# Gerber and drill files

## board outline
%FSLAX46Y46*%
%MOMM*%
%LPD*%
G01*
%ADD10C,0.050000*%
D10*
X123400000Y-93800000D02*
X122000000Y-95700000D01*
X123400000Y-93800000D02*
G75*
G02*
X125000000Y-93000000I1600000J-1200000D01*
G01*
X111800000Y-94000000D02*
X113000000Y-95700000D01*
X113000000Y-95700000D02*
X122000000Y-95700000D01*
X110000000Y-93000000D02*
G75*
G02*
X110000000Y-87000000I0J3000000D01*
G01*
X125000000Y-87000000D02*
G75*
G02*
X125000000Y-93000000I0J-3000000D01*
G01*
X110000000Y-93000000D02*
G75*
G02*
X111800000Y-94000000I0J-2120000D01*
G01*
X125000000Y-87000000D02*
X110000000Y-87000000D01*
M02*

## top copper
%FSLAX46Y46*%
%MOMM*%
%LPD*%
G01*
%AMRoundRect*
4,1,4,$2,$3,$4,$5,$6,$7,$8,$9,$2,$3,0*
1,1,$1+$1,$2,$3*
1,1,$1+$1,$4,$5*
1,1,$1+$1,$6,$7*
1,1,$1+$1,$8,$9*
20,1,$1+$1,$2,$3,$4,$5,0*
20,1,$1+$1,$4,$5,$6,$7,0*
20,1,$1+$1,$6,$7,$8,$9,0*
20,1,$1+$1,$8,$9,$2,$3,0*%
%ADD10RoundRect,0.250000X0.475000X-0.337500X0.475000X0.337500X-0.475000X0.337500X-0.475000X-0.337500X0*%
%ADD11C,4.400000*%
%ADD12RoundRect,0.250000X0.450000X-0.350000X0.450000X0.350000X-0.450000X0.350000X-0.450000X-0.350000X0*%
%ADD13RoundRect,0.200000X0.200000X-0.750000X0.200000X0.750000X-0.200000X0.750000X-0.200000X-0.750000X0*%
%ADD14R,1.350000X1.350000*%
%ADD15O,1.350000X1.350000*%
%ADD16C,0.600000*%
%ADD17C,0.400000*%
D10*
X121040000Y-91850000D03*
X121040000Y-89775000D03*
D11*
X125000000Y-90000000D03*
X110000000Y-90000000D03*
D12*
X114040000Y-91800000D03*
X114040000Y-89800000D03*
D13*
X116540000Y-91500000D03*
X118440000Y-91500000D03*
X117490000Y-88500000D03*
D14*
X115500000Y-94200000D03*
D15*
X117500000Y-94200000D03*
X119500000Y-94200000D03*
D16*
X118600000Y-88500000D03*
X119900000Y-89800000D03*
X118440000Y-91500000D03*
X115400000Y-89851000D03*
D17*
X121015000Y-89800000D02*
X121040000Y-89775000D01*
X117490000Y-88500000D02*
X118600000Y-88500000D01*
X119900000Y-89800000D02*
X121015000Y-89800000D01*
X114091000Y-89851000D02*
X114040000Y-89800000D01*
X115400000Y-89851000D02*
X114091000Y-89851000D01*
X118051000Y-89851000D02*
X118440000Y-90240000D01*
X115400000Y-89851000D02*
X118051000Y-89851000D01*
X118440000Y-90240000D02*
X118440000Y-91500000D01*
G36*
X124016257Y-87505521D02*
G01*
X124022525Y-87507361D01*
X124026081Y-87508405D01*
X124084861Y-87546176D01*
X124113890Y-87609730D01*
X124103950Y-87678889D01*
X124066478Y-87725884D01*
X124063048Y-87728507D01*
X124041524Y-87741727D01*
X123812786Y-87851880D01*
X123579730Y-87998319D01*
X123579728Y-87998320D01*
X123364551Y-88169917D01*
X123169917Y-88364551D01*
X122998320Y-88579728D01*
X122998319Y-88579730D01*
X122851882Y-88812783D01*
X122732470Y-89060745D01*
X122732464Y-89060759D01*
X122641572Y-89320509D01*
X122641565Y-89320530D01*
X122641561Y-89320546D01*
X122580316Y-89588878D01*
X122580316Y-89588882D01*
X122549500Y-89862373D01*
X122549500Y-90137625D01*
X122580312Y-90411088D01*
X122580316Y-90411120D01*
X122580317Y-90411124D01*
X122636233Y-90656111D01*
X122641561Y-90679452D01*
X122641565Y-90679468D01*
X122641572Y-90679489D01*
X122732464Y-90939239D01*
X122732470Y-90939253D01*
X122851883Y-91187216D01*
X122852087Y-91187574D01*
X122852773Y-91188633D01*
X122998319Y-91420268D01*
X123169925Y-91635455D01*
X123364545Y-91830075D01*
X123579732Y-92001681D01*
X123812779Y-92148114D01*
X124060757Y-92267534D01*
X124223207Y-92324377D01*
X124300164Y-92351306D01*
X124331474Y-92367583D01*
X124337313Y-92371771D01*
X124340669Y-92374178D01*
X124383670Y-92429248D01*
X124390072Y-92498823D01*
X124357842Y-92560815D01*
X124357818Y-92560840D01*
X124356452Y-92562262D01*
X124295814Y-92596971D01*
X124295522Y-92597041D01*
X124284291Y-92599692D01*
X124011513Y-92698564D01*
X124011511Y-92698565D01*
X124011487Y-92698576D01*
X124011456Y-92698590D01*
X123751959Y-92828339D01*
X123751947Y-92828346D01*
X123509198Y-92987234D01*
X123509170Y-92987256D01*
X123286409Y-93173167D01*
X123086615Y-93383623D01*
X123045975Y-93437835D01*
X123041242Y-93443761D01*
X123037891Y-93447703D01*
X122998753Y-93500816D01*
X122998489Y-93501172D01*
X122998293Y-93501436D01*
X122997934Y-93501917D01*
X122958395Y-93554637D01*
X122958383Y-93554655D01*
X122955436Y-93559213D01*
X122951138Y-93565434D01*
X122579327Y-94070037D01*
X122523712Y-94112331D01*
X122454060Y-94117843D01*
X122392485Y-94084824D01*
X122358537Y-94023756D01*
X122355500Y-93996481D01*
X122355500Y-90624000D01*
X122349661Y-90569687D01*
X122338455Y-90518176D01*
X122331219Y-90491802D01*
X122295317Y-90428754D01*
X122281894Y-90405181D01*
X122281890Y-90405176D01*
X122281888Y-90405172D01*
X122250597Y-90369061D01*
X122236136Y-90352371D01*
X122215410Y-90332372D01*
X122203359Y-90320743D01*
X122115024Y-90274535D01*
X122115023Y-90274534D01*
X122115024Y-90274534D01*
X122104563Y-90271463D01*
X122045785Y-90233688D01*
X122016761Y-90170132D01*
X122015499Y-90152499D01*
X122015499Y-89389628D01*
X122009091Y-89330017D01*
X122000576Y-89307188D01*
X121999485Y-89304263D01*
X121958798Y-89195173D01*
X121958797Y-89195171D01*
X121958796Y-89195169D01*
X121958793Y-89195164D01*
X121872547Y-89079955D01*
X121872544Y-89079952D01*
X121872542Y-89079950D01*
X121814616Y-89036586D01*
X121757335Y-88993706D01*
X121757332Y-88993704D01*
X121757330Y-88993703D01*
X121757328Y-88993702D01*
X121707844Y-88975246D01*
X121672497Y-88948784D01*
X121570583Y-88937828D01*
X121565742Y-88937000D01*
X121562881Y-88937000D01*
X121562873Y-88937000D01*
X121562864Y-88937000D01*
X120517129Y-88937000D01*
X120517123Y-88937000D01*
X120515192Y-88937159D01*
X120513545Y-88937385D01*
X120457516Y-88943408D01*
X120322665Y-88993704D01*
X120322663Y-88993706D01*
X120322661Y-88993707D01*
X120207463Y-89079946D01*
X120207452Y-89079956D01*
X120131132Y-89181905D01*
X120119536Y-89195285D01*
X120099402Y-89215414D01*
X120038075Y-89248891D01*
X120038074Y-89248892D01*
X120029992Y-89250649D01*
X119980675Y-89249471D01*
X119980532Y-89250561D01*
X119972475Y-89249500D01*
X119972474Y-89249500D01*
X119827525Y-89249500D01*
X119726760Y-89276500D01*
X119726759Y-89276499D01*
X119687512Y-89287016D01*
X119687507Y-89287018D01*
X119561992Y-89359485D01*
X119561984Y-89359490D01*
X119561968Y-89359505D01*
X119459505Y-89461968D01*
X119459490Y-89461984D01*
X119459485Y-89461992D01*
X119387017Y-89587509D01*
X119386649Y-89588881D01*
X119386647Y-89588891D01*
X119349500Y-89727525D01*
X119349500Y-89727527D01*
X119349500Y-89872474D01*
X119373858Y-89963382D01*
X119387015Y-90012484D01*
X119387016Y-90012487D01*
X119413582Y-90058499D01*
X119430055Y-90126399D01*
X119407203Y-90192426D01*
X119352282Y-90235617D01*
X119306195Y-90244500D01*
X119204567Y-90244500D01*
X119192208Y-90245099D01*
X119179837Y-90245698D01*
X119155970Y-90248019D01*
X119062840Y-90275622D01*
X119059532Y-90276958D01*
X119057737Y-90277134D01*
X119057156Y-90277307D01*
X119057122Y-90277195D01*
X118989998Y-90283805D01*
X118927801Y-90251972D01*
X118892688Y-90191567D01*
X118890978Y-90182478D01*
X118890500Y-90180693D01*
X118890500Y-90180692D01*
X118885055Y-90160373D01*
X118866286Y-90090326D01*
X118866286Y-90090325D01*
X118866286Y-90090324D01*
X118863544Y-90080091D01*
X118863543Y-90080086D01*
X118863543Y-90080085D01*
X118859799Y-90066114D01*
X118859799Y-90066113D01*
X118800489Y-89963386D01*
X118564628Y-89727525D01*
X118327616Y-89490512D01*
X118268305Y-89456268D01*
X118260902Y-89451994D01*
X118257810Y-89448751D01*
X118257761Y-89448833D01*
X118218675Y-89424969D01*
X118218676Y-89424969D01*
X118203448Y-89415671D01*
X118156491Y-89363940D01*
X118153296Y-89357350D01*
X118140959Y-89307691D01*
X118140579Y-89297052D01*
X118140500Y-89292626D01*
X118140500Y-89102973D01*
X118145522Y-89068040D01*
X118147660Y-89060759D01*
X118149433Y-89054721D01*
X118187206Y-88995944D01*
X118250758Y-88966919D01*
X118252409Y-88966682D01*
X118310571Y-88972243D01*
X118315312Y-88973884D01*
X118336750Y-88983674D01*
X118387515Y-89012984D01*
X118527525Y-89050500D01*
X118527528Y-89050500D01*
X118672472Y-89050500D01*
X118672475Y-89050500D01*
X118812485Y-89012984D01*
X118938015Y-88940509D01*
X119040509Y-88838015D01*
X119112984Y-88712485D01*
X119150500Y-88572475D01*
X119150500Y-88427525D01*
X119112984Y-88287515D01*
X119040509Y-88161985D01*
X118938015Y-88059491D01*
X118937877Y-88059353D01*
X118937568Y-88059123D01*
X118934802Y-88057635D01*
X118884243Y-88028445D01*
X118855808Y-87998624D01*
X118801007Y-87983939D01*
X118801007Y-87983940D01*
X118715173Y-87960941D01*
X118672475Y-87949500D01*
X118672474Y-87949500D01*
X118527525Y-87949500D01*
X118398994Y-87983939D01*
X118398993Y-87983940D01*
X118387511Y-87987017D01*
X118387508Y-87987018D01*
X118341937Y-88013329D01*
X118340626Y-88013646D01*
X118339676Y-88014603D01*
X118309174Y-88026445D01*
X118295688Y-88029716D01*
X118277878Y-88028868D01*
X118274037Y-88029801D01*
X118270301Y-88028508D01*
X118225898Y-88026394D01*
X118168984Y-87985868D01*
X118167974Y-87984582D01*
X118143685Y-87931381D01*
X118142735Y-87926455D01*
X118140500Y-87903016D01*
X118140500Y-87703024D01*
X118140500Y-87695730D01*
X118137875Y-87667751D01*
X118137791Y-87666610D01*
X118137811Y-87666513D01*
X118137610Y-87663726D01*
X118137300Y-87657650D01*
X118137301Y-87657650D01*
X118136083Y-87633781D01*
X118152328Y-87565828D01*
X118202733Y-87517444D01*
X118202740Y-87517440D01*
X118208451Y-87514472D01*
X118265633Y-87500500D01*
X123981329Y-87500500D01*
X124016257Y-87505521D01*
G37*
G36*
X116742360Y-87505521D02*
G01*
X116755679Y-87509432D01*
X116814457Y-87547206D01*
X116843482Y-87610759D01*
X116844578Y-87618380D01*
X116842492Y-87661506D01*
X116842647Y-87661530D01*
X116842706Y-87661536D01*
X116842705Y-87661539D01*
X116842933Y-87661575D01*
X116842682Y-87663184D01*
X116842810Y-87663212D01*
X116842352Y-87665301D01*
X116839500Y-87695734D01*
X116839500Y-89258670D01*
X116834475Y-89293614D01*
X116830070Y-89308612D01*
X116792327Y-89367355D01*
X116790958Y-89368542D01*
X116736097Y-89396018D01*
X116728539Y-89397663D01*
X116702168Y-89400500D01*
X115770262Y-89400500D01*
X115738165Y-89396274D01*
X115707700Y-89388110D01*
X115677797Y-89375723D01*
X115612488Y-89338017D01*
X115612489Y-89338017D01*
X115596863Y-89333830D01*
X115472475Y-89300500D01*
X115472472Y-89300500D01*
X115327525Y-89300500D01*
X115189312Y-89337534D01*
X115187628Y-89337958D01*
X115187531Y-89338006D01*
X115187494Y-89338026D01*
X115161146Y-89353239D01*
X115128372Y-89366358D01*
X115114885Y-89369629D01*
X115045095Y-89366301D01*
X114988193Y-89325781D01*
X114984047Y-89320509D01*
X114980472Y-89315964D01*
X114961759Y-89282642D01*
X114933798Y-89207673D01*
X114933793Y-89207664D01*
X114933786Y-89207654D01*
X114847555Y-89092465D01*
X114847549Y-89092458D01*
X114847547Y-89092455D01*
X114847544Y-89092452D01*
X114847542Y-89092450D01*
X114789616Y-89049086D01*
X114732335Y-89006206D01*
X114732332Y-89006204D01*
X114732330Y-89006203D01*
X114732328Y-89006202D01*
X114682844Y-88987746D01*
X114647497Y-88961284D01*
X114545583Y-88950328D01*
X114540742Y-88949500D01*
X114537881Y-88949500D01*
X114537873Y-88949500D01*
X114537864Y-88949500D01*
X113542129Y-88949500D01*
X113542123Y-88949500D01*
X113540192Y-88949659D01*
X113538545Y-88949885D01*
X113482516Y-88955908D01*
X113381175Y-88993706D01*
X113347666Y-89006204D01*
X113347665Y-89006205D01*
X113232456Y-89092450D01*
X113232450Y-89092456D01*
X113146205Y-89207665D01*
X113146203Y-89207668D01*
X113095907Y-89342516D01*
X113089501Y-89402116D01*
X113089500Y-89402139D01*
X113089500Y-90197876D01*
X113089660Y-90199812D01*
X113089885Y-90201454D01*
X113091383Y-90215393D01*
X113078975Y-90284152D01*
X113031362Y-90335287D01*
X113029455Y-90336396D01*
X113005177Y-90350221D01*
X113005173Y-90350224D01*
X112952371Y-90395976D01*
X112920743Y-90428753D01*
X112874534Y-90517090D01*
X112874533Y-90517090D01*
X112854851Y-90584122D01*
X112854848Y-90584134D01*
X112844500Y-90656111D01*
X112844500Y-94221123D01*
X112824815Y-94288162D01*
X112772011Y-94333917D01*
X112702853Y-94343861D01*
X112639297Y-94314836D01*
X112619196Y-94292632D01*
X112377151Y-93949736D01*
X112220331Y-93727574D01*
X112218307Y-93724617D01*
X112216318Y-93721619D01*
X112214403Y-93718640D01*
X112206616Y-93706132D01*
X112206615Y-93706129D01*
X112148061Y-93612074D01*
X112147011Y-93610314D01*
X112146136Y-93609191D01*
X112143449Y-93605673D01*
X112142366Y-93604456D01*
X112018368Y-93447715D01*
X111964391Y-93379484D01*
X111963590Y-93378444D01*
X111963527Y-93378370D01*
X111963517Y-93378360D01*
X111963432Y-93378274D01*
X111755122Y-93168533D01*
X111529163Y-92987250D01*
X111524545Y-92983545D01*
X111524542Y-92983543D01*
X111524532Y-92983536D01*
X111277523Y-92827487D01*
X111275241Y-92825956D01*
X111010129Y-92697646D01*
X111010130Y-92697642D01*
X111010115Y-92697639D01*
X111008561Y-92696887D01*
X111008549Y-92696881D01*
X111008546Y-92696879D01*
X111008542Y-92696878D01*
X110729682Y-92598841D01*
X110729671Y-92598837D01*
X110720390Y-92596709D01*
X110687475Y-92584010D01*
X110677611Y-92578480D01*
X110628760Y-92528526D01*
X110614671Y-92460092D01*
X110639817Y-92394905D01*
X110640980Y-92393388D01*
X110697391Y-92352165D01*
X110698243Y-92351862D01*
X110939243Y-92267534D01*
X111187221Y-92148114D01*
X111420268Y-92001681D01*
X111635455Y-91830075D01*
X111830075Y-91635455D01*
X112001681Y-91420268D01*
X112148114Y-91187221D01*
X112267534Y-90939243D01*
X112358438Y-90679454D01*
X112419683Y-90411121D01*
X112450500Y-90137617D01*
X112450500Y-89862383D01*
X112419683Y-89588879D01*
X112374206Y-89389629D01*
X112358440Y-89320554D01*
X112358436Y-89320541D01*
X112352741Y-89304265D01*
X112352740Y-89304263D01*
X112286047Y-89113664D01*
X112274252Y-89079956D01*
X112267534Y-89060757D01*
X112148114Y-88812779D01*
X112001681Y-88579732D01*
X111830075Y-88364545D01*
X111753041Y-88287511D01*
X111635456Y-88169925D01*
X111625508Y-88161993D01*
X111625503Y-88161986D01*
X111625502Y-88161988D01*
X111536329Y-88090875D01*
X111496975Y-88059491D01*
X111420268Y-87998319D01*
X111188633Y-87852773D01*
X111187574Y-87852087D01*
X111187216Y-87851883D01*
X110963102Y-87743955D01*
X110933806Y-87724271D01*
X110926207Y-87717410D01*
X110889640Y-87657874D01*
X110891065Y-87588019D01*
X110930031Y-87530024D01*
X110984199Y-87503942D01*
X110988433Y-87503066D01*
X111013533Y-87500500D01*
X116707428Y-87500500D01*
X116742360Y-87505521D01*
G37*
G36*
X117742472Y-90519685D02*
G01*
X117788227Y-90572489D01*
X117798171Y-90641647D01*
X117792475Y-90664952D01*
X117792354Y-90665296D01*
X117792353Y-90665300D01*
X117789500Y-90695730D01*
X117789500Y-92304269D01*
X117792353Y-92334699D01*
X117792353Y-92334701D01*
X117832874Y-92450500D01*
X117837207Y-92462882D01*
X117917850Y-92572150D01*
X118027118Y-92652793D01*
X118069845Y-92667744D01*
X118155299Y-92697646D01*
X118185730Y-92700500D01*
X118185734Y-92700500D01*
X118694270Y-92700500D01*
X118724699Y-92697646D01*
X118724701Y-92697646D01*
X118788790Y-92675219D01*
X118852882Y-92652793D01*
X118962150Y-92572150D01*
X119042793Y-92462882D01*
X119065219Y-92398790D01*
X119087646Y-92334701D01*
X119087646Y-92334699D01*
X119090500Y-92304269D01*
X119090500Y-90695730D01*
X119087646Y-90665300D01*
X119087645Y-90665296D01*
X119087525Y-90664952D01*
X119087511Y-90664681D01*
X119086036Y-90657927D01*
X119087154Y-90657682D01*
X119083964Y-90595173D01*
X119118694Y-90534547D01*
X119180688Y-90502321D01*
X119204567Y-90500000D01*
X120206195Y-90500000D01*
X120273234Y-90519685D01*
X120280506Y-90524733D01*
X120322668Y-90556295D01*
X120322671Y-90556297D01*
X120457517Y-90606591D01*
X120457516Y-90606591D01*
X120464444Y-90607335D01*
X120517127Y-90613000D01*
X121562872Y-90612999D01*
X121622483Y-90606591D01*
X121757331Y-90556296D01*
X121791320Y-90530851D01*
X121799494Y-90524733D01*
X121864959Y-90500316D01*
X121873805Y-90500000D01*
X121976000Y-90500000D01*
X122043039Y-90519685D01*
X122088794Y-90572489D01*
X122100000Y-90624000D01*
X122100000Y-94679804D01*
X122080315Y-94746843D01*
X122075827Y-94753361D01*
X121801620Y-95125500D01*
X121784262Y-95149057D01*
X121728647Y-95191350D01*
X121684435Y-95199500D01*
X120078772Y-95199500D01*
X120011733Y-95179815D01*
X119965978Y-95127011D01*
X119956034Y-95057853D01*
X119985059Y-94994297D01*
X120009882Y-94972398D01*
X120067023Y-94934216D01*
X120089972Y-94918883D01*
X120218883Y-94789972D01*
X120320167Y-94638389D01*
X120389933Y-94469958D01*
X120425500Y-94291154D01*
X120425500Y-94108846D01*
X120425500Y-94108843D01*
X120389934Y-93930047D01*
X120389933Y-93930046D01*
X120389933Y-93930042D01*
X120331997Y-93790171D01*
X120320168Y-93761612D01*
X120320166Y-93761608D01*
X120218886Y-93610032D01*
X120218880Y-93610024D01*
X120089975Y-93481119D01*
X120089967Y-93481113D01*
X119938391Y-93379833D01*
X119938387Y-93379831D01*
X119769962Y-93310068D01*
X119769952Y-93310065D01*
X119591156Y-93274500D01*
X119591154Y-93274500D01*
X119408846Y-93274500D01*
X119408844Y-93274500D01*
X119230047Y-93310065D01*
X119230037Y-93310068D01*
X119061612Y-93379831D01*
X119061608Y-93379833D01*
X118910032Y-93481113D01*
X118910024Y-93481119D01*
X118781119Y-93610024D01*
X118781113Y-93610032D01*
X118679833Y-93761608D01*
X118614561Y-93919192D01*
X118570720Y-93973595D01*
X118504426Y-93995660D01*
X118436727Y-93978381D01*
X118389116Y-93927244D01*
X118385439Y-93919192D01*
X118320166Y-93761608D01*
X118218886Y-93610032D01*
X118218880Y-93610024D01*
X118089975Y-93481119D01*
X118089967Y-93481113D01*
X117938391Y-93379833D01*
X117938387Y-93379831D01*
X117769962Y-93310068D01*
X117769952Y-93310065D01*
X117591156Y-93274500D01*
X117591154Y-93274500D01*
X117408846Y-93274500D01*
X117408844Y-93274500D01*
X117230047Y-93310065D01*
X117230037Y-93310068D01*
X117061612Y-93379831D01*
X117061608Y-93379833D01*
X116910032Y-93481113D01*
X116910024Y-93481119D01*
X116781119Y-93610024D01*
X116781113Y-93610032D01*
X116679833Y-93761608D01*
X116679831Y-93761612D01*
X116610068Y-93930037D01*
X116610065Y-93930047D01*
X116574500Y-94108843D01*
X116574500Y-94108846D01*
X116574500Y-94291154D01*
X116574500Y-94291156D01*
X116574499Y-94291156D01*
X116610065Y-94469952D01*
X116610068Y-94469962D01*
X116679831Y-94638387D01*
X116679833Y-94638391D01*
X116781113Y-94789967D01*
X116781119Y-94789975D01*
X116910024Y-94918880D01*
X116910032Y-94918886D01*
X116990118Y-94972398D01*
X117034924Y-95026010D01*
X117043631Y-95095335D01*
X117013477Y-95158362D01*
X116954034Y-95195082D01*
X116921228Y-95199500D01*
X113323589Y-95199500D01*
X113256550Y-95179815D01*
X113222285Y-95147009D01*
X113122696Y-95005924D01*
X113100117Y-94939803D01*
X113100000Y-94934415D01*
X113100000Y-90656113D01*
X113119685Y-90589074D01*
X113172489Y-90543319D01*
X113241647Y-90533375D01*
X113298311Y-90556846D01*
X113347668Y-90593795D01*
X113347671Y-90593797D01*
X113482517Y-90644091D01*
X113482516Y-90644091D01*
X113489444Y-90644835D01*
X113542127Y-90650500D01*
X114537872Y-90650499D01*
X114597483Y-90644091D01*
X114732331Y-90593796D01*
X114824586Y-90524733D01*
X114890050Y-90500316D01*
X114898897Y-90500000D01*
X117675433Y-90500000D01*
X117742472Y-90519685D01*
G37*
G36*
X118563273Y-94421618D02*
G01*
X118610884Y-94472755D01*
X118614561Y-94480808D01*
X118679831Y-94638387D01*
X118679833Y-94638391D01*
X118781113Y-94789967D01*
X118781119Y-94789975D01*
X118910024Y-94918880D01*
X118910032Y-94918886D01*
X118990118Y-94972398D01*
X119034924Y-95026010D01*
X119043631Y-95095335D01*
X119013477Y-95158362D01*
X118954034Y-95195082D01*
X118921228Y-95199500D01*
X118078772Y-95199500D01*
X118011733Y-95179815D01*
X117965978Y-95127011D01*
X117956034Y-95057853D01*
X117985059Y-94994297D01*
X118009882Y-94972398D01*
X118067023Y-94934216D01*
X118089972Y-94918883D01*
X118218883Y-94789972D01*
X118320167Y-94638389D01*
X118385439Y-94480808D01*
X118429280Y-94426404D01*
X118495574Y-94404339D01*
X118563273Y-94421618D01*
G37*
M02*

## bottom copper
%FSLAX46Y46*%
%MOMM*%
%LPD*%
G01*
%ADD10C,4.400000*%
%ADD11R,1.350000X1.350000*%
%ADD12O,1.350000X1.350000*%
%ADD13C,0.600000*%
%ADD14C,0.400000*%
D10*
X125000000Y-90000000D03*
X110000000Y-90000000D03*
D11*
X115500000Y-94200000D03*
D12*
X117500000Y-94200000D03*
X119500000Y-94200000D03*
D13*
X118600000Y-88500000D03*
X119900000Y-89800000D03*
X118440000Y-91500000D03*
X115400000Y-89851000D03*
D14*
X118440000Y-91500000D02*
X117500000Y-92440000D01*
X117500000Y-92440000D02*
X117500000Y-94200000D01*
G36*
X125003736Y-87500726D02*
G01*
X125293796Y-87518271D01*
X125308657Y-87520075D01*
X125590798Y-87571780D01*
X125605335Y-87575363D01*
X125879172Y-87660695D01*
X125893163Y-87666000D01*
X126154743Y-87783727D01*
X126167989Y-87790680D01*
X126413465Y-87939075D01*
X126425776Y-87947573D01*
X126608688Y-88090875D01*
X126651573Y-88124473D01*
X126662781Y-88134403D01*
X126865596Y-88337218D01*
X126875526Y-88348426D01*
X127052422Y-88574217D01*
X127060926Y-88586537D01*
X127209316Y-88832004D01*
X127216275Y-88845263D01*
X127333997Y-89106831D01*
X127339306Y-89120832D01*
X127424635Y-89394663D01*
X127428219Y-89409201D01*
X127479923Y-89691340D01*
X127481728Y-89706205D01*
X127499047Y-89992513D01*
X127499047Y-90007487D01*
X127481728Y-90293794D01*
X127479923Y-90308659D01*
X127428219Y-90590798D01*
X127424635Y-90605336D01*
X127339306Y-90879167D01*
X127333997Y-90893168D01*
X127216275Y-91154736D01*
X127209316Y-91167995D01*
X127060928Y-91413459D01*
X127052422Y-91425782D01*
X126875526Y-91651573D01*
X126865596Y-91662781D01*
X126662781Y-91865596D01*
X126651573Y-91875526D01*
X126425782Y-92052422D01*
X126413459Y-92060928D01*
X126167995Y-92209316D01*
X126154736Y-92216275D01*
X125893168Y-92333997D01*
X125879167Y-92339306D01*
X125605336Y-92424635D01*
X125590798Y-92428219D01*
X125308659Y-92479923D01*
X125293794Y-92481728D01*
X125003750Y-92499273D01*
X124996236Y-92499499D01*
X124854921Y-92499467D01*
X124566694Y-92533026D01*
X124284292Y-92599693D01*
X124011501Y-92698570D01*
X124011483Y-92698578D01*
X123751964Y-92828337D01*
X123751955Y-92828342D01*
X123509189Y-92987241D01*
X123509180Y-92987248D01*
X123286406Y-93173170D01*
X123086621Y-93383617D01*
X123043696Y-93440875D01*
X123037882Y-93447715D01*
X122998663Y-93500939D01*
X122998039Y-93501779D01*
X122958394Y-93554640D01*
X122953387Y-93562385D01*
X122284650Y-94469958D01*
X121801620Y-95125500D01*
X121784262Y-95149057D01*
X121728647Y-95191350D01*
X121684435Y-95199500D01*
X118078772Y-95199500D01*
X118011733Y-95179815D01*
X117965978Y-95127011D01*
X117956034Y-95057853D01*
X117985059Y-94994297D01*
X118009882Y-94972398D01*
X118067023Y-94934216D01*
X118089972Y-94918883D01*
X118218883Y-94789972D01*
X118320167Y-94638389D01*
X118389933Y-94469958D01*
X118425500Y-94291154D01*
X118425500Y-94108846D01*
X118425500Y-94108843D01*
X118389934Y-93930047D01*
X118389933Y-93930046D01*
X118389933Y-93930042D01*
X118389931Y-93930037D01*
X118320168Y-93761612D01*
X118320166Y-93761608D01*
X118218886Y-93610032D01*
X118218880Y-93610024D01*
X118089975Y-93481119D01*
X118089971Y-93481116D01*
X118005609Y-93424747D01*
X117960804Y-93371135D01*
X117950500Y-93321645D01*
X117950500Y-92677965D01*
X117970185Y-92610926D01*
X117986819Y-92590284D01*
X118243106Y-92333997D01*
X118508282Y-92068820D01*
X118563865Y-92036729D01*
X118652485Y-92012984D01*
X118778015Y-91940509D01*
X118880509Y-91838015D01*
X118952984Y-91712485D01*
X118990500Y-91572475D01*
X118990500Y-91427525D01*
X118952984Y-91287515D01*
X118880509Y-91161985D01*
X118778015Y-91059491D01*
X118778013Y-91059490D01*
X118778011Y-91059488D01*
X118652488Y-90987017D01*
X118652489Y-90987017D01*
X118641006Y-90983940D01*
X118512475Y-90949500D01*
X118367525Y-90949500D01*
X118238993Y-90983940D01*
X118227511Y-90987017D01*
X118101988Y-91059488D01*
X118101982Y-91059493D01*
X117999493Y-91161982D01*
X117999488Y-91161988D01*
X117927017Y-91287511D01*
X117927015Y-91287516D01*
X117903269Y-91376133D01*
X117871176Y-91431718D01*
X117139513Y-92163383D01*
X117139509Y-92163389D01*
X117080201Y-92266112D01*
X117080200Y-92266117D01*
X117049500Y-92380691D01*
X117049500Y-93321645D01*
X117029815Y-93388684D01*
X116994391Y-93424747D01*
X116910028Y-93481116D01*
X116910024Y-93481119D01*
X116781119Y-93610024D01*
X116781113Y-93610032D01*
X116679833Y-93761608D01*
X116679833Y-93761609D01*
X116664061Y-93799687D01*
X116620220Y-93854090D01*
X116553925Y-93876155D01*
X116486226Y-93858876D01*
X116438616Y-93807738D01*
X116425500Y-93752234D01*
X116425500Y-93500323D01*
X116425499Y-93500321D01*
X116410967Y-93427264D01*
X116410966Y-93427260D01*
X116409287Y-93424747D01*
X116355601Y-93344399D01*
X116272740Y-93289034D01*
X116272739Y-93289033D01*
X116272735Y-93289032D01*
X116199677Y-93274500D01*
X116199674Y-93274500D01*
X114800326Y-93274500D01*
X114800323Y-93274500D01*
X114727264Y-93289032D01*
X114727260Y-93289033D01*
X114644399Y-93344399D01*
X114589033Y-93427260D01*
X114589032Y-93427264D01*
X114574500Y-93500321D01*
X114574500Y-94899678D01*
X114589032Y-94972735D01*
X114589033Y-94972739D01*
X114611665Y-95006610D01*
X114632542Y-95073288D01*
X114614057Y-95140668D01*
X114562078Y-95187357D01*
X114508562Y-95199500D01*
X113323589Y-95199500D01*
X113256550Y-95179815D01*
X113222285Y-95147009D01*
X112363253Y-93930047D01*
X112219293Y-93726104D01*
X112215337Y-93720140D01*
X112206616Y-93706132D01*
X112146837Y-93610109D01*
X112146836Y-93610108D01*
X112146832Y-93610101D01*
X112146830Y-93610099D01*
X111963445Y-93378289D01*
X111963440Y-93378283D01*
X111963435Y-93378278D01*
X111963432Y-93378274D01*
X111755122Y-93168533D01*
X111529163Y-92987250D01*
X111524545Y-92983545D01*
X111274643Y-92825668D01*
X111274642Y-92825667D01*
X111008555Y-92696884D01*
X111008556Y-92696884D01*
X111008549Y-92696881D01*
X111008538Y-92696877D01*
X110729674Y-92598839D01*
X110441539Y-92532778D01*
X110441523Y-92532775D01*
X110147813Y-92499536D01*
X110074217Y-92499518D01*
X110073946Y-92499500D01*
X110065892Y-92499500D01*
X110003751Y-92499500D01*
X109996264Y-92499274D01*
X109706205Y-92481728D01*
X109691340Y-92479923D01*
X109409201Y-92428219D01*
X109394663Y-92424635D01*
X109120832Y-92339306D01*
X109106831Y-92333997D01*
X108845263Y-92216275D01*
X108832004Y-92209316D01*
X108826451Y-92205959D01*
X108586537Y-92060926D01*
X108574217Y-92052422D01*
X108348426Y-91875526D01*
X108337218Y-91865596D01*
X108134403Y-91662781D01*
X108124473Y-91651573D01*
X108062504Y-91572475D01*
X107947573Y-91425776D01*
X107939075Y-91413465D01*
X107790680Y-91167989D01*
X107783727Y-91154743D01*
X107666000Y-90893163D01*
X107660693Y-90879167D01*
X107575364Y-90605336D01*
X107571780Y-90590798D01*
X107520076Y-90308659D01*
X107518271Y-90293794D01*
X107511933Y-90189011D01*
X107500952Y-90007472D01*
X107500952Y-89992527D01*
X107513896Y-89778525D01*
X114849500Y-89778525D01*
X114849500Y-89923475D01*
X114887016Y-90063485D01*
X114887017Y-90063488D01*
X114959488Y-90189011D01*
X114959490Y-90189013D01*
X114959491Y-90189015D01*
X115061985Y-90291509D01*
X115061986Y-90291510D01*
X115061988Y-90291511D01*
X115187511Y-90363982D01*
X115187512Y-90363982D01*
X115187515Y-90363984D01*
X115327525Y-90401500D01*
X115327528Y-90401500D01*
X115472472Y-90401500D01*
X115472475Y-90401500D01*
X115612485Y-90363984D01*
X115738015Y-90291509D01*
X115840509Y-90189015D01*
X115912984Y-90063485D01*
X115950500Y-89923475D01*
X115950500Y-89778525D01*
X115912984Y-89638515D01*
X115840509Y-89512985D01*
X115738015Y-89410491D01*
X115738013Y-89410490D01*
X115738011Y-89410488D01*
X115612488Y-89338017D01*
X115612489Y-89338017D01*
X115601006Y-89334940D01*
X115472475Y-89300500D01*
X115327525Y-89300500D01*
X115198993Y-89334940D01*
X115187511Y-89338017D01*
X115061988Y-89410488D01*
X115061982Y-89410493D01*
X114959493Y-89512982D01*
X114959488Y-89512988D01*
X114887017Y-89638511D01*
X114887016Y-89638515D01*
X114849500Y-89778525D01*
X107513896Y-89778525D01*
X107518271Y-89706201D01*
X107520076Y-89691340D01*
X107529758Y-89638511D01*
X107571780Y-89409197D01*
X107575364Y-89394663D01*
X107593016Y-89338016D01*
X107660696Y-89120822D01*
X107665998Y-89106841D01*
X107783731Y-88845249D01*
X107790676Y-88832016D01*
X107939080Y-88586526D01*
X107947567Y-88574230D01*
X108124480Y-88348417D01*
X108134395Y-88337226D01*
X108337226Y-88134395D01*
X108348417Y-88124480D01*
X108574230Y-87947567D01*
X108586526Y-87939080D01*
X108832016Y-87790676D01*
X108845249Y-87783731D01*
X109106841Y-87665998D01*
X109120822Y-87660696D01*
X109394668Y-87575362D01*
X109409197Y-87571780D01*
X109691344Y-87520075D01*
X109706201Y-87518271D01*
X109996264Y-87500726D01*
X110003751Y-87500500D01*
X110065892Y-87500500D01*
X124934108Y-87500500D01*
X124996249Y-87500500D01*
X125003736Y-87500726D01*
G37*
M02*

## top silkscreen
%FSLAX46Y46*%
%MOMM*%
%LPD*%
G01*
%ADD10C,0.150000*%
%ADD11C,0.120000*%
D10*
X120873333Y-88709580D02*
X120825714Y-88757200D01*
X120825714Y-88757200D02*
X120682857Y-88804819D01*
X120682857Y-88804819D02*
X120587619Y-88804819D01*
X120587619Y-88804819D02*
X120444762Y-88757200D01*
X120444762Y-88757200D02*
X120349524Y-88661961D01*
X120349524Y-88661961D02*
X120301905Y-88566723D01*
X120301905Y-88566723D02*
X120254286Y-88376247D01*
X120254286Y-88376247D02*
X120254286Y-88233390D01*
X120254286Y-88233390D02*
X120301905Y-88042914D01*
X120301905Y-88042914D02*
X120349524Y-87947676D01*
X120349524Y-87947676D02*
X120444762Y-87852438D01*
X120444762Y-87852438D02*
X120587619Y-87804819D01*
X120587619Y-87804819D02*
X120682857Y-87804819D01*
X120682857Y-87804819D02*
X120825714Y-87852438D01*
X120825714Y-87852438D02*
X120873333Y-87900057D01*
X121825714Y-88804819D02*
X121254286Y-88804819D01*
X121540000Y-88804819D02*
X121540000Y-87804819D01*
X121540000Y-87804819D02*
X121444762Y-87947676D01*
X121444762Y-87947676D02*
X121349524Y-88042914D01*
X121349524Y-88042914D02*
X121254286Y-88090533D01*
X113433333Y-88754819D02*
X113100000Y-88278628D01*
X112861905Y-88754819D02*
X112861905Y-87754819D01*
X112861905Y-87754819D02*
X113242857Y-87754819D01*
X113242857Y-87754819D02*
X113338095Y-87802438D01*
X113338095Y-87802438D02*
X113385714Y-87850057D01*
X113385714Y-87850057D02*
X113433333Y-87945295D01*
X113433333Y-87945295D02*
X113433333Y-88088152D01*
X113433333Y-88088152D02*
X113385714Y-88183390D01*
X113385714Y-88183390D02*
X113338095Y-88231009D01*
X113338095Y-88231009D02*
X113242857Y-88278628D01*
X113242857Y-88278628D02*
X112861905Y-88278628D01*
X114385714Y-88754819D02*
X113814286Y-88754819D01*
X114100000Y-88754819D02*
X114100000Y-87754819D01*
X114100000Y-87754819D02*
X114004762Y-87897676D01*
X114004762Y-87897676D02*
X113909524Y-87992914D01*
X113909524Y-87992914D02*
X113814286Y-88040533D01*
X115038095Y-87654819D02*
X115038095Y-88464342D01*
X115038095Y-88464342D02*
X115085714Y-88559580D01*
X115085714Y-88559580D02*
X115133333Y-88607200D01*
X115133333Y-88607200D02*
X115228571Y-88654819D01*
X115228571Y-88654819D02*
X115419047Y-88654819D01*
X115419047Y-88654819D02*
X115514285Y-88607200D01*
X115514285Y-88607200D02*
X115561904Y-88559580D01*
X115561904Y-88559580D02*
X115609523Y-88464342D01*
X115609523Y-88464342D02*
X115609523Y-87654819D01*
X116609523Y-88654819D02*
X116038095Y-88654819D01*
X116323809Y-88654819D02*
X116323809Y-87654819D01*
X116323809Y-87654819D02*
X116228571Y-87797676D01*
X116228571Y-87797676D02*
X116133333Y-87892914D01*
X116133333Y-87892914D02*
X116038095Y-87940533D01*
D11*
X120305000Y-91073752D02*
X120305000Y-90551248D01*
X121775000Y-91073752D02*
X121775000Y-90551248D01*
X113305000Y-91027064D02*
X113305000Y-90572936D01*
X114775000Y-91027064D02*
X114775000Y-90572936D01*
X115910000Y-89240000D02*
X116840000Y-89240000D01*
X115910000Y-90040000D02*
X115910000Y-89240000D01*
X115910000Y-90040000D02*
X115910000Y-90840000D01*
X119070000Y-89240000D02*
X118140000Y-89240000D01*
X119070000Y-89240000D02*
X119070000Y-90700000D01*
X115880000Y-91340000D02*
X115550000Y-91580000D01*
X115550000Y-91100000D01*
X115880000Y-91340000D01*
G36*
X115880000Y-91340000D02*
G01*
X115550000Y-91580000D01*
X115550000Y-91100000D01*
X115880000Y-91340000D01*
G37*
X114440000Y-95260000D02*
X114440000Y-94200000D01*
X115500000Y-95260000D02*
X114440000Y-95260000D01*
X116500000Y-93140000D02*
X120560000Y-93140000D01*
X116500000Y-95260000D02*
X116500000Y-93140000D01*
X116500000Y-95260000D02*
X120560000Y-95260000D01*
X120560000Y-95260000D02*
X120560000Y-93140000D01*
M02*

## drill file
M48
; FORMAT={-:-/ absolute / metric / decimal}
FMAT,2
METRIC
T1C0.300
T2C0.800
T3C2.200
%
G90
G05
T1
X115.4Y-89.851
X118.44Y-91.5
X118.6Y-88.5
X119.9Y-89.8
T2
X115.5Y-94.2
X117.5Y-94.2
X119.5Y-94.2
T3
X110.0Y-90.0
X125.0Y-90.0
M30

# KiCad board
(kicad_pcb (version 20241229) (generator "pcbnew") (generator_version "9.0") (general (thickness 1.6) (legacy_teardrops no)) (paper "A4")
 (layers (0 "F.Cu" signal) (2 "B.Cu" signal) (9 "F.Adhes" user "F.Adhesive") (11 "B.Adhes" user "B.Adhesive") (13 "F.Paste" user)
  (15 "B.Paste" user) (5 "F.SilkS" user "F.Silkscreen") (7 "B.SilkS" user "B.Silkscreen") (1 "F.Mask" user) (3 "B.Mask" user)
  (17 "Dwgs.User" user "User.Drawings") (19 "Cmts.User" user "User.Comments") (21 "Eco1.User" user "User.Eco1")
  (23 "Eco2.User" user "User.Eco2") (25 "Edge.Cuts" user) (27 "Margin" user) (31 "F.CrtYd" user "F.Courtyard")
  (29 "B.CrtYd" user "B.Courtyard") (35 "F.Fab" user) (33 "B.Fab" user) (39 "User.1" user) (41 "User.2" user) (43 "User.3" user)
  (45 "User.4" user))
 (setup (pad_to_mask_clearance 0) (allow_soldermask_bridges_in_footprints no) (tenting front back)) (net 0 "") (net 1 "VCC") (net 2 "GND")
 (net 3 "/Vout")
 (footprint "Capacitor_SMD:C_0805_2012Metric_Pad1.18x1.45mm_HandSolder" (layer "F.Cu") (at 121.04 90.8125 90)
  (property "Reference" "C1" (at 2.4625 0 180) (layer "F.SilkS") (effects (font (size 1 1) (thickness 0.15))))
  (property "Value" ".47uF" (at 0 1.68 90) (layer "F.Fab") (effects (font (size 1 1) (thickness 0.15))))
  (fp_line (start -0.261252 -0.735) (end 0.261252 -0.735) (stroke (width 0.12) (type solid)) (layer "F.SilkS"))
  (fp_line (start -0.261252 0.735) (end 0.261252 0.735) (stroke (width 0.12) (type solid)) (layer "F.SilkS"))
  (pad "1" smd roundrect (at -1.0375 0 90) (size 1.175 1.45) (layers "F.Cu" "F.Mask" "F.Paste") (roundrect_rratio 0.212766) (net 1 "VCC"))
  (pad "2" smd roundrect (at 1.0375 0 90) (size 1.175 1.45) (layers "F.Cu" "F.Mask" "F.Paste") (roundrect_rratio 0.212766) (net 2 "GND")))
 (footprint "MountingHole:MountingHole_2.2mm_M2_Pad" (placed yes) (layer "F.Cu") (at 125 90)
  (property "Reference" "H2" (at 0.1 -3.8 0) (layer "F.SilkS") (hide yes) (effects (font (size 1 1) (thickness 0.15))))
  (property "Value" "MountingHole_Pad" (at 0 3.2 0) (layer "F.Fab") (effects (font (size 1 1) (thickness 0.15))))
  (pad "1" thru_hole circle (at 0 0) (size 4.4 4.4) (drill 2.2) (layers "*.Cu" "*.Mask") (remove_unused_layers no) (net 2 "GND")))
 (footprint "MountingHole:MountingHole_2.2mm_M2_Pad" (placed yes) (layer "F.Cu") (at 110 90)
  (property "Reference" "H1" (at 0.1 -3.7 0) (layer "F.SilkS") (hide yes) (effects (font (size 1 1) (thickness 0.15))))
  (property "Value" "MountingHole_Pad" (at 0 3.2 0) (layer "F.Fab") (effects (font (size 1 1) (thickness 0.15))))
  (pad "1" thru_hole circle (at 0 0) (size 4.4 4.4) (drill 2.2) (layers "*.Cu" "*.Mask") (remove_unused_layers no) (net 2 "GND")))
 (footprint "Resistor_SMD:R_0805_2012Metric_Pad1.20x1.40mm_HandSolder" (layer "F.Cu") (at 114.04 90.8 90)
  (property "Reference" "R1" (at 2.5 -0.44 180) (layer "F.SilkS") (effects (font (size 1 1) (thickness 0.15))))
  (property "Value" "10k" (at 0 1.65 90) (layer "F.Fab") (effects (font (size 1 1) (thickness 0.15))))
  (fp_line (start -0.227064 -0.735) (end 0.227064 -0.735) (stroke (width 0.12) (type solid)) (layer "F.SilkS"))
  (fp_line (start -0.227064 0.735) (end 0.227064 0.735) (stroke (width 0.12) (type solid)) (layer "F.SilkS"))
  (pad "1" smd roundrect (at -1 0 90) (size 1.2 1.4) (layers "F.Cu" "F.Mask" "F.Paste") (roundrect_rratio 0.208333) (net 1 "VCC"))
  (pad "2" smd roundrect (at 1 0 90) (size 1.2 1.4) (layers "F.Cu" "F.Mask" "F.Paste") (roundrect_rratio 0.208333) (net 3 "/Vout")))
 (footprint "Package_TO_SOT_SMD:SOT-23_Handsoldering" (layer "F.Cu") (at 117.49 90 90)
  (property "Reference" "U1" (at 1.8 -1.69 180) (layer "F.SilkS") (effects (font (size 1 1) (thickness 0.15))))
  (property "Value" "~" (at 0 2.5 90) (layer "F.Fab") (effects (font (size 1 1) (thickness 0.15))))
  (fp_line (start 0.76 -1.58) (end 0.76 -0.65) (stroke (width 0.12) (type solid)) (layer "F.SilkS"))
  (fp_line (start -0.04 -1.58) (end 0.76 -1.58) (stroke (width 0.12) (type solid)) (layer "F.SilkS"))
  (fp_line (start -0.04 -1.58) (end -0.84 -1.58) (stroke (width 0.12) (type solid)) (layer "F.SilkS"))
  (fp_line (start 0.76 1.58) (end 0.76 0.65) (stroke (width 0.12) (type solid)) (layer "F.SilkS"))
  (fp_line (start 0.76 1.58) (end -0.7 1.58) (stroke (width 0.12) (type solid)) (layer "F.SilkS"))
  (fp_poly
   (pts (xy -1.34 -1.61) (xy -1.58 -1.94) (xy -1.1 -1.94) (xy -1.34 -1.61)) (stroke (width 0.12) (type solid)) (fill yes) (layer "F.SilkS"))
  (pad "1" smd roundrect (at -1.5 -0.95 90) (size 1.9 0.8) (layers "F.Cu" "F.Mask" "F.Paste") (roundrect_rratio 0.25) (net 1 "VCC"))
  (pad "2" smd roundrect (at -1.5 0.95 90) (size 1.9 0.8) (layers "F.Cu" "F.Mask" "F.Paste") (roundrect_rratio 0.25) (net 3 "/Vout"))
  (pad "3" smd roundrect (at 1.5 0 90) (size 1.9 0.8) (layers "F.Cu" "F.Mask" "F.Paste") (roundrect_rratio 0.25) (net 2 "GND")))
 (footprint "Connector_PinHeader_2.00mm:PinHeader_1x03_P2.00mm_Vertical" (layer "F.Cu") (at 115.5 94.2 90)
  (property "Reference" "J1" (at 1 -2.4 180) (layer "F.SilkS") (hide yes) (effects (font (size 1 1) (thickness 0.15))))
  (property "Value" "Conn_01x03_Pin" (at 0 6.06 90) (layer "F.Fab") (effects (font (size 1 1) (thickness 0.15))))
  (fp_line (start -1.06 -1.06) (end 0 -1.06) (stroke (width 0.12) (type solid)) (layer "F.SilkS"))
  (fp_line (start -1.06 0) (end -1.06 -1.06) (stroke (width 0.12) (type solid)) (layer "F.SilkS"))
  (fp_line (start 1.06 1) (end 1.06 5.06) (stroke (width 0.12) (type solid)) (layer "F.SilkS"))
  (fp_line (start -1.06 1) (end 1.06 1) (stroke (width 0.12) (type solid)) (layer "F.SilkS"))
  (fp_line (start -1.06 1) (end -1.06 5.06) (stroke (width 0.12) (type solid)) (layer "F.SilkS"))
  (fp_line (start -1.06 5.06) (end 1.06 5.06) (stroke (width 0.12) (type solid)) (layer "F.SilkS"))
  (pad "1" thru_hole rect (at 0 0 90) (size 1.35 1.35) (drill 0.8) (layers "*.Cu" "*.Mask") (remove_unused_layers no) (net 1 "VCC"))
  (pad "2" thru_hole oval (at 0 2 90) (size 1.35 1.35) (drill 0.8) (layers "*.Cu" "*.Mask") (remove_unused_layers no) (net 3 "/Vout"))
  (pad "3" thru_hole oval (at 0 4 90) (size 1.35 1.35) (drill 0.8) (layers "*.Cu" "*.Mask") (remove_unused_layers no) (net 2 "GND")))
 (gr_line (start 123.4 93.8) (end 122 95.7) (stroke (width 0.05) (type default)) (layer "Edge.Cuts"))
 (gr_arc (start 123.4 93.8) (mid 124.105573 93.211146) (end 125 93) (stroke (width 0.05) (type default)) (layer "Edge.Cuts"))
 (gr_line (start 111.8 94) (end 113 95.7) (stroke (width 0.05) (type default)) (layer "Edge.Cuts"))
 (gr_line (start 113 95.7) (end 122 95.7) (stroke (width 0.05) (type default)) (layer "Edge.Cuts"))
 (gr_arc (start 110 93) (mid 107 90) (end 110 87) (stroke (width 0.05) (type default)) (layer "Edge.Cuts"))
 (gr_arc (start 125 87) (mid 128 90) (end 125 93) (stroke (width 0.05) (type default)) (layer "Edge.Cuts"))
 (gr_arc (start 110 93) (mid 111.029563 93.266787) (end 111.8 94) (stroke (width 0.05) (type default)) (layer "Edge.Cuts"))
 (gr_line (start 125 87) (end 110 87) (stroke (width 0.05) (type default)) (layer "Edge.Cuts"))
 (segment (start 121.015 89.8) (end 121.04 89.775) (width 0.4) (layer "F.Cu") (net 2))
 (segment (start 117.49 88.5) (end 118.6 88.5) (width 0.4) (layer "F.Cu") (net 2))
 (segment (start 119.9 89.8) (end 121.015 89.8) (width 0.4) (layer "F.Cu") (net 2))
 (via (at 118.6 88.5) (size 0.6) (drill 0.3) (layers "F.Cu" "B.Cu") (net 2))
 (via (at 119.9 89.8) (size 0.6) (drill 0.3) (layers "F.Cu" "B.Cu") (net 2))
 (segment (start 114.091 89.851) (end 114.04 89.8) (width 0.4) (layer "F.Cu") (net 3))
 (segment (start 115.4 89.851) (end 114.091 89.851) (width 0.4) (layer "F.Cu") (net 3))
 (segment (start 118.051 89.851) (end 118.44 90.24) (width 0.4) (layer "F.Cu") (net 3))
 (segment (start 115.4 89.851) (end 118.051 89.851) (width 0.4) (layer "F.Cu") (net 3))
 (segment (start 118.44 90.24) (end 118.44 91.5) (width 0.4) (layer "F.Cu") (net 3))
 (via (at 118.44 91.5) (size 0.6) (drill 0.3) (layers "F.Cu" "B.Cu") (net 3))
 (via (at 115.4 89.851) (size 0.6) (drill 0.3) (layers "F.Cu" "B.Cu") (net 3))
 (segment (start 118.44 91.5) (end 117.5 92.44) (width 0.4) (layer "B.Cu") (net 3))
 (segment (start 117.5 92.44) (end 117.5 94.2) (width 0.4) (layer "B.Cu") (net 3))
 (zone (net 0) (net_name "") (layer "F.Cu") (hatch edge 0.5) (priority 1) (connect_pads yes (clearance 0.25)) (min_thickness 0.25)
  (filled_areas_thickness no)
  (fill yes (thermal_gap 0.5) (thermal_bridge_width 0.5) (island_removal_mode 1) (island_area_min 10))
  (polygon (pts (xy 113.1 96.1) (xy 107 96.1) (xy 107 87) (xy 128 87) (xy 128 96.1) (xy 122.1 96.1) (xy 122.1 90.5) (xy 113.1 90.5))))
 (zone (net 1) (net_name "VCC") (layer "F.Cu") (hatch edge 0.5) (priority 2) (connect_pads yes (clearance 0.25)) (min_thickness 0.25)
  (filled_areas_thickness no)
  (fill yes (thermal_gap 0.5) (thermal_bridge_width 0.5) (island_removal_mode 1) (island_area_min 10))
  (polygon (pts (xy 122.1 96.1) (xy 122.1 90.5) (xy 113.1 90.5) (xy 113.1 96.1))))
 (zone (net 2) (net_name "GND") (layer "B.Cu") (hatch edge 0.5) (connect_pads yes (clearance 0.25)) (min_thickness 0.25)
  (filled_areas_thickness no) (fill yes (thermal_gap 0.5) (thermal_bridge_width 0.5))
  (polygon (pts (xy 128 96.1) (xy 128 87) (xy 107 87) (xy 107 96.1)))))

